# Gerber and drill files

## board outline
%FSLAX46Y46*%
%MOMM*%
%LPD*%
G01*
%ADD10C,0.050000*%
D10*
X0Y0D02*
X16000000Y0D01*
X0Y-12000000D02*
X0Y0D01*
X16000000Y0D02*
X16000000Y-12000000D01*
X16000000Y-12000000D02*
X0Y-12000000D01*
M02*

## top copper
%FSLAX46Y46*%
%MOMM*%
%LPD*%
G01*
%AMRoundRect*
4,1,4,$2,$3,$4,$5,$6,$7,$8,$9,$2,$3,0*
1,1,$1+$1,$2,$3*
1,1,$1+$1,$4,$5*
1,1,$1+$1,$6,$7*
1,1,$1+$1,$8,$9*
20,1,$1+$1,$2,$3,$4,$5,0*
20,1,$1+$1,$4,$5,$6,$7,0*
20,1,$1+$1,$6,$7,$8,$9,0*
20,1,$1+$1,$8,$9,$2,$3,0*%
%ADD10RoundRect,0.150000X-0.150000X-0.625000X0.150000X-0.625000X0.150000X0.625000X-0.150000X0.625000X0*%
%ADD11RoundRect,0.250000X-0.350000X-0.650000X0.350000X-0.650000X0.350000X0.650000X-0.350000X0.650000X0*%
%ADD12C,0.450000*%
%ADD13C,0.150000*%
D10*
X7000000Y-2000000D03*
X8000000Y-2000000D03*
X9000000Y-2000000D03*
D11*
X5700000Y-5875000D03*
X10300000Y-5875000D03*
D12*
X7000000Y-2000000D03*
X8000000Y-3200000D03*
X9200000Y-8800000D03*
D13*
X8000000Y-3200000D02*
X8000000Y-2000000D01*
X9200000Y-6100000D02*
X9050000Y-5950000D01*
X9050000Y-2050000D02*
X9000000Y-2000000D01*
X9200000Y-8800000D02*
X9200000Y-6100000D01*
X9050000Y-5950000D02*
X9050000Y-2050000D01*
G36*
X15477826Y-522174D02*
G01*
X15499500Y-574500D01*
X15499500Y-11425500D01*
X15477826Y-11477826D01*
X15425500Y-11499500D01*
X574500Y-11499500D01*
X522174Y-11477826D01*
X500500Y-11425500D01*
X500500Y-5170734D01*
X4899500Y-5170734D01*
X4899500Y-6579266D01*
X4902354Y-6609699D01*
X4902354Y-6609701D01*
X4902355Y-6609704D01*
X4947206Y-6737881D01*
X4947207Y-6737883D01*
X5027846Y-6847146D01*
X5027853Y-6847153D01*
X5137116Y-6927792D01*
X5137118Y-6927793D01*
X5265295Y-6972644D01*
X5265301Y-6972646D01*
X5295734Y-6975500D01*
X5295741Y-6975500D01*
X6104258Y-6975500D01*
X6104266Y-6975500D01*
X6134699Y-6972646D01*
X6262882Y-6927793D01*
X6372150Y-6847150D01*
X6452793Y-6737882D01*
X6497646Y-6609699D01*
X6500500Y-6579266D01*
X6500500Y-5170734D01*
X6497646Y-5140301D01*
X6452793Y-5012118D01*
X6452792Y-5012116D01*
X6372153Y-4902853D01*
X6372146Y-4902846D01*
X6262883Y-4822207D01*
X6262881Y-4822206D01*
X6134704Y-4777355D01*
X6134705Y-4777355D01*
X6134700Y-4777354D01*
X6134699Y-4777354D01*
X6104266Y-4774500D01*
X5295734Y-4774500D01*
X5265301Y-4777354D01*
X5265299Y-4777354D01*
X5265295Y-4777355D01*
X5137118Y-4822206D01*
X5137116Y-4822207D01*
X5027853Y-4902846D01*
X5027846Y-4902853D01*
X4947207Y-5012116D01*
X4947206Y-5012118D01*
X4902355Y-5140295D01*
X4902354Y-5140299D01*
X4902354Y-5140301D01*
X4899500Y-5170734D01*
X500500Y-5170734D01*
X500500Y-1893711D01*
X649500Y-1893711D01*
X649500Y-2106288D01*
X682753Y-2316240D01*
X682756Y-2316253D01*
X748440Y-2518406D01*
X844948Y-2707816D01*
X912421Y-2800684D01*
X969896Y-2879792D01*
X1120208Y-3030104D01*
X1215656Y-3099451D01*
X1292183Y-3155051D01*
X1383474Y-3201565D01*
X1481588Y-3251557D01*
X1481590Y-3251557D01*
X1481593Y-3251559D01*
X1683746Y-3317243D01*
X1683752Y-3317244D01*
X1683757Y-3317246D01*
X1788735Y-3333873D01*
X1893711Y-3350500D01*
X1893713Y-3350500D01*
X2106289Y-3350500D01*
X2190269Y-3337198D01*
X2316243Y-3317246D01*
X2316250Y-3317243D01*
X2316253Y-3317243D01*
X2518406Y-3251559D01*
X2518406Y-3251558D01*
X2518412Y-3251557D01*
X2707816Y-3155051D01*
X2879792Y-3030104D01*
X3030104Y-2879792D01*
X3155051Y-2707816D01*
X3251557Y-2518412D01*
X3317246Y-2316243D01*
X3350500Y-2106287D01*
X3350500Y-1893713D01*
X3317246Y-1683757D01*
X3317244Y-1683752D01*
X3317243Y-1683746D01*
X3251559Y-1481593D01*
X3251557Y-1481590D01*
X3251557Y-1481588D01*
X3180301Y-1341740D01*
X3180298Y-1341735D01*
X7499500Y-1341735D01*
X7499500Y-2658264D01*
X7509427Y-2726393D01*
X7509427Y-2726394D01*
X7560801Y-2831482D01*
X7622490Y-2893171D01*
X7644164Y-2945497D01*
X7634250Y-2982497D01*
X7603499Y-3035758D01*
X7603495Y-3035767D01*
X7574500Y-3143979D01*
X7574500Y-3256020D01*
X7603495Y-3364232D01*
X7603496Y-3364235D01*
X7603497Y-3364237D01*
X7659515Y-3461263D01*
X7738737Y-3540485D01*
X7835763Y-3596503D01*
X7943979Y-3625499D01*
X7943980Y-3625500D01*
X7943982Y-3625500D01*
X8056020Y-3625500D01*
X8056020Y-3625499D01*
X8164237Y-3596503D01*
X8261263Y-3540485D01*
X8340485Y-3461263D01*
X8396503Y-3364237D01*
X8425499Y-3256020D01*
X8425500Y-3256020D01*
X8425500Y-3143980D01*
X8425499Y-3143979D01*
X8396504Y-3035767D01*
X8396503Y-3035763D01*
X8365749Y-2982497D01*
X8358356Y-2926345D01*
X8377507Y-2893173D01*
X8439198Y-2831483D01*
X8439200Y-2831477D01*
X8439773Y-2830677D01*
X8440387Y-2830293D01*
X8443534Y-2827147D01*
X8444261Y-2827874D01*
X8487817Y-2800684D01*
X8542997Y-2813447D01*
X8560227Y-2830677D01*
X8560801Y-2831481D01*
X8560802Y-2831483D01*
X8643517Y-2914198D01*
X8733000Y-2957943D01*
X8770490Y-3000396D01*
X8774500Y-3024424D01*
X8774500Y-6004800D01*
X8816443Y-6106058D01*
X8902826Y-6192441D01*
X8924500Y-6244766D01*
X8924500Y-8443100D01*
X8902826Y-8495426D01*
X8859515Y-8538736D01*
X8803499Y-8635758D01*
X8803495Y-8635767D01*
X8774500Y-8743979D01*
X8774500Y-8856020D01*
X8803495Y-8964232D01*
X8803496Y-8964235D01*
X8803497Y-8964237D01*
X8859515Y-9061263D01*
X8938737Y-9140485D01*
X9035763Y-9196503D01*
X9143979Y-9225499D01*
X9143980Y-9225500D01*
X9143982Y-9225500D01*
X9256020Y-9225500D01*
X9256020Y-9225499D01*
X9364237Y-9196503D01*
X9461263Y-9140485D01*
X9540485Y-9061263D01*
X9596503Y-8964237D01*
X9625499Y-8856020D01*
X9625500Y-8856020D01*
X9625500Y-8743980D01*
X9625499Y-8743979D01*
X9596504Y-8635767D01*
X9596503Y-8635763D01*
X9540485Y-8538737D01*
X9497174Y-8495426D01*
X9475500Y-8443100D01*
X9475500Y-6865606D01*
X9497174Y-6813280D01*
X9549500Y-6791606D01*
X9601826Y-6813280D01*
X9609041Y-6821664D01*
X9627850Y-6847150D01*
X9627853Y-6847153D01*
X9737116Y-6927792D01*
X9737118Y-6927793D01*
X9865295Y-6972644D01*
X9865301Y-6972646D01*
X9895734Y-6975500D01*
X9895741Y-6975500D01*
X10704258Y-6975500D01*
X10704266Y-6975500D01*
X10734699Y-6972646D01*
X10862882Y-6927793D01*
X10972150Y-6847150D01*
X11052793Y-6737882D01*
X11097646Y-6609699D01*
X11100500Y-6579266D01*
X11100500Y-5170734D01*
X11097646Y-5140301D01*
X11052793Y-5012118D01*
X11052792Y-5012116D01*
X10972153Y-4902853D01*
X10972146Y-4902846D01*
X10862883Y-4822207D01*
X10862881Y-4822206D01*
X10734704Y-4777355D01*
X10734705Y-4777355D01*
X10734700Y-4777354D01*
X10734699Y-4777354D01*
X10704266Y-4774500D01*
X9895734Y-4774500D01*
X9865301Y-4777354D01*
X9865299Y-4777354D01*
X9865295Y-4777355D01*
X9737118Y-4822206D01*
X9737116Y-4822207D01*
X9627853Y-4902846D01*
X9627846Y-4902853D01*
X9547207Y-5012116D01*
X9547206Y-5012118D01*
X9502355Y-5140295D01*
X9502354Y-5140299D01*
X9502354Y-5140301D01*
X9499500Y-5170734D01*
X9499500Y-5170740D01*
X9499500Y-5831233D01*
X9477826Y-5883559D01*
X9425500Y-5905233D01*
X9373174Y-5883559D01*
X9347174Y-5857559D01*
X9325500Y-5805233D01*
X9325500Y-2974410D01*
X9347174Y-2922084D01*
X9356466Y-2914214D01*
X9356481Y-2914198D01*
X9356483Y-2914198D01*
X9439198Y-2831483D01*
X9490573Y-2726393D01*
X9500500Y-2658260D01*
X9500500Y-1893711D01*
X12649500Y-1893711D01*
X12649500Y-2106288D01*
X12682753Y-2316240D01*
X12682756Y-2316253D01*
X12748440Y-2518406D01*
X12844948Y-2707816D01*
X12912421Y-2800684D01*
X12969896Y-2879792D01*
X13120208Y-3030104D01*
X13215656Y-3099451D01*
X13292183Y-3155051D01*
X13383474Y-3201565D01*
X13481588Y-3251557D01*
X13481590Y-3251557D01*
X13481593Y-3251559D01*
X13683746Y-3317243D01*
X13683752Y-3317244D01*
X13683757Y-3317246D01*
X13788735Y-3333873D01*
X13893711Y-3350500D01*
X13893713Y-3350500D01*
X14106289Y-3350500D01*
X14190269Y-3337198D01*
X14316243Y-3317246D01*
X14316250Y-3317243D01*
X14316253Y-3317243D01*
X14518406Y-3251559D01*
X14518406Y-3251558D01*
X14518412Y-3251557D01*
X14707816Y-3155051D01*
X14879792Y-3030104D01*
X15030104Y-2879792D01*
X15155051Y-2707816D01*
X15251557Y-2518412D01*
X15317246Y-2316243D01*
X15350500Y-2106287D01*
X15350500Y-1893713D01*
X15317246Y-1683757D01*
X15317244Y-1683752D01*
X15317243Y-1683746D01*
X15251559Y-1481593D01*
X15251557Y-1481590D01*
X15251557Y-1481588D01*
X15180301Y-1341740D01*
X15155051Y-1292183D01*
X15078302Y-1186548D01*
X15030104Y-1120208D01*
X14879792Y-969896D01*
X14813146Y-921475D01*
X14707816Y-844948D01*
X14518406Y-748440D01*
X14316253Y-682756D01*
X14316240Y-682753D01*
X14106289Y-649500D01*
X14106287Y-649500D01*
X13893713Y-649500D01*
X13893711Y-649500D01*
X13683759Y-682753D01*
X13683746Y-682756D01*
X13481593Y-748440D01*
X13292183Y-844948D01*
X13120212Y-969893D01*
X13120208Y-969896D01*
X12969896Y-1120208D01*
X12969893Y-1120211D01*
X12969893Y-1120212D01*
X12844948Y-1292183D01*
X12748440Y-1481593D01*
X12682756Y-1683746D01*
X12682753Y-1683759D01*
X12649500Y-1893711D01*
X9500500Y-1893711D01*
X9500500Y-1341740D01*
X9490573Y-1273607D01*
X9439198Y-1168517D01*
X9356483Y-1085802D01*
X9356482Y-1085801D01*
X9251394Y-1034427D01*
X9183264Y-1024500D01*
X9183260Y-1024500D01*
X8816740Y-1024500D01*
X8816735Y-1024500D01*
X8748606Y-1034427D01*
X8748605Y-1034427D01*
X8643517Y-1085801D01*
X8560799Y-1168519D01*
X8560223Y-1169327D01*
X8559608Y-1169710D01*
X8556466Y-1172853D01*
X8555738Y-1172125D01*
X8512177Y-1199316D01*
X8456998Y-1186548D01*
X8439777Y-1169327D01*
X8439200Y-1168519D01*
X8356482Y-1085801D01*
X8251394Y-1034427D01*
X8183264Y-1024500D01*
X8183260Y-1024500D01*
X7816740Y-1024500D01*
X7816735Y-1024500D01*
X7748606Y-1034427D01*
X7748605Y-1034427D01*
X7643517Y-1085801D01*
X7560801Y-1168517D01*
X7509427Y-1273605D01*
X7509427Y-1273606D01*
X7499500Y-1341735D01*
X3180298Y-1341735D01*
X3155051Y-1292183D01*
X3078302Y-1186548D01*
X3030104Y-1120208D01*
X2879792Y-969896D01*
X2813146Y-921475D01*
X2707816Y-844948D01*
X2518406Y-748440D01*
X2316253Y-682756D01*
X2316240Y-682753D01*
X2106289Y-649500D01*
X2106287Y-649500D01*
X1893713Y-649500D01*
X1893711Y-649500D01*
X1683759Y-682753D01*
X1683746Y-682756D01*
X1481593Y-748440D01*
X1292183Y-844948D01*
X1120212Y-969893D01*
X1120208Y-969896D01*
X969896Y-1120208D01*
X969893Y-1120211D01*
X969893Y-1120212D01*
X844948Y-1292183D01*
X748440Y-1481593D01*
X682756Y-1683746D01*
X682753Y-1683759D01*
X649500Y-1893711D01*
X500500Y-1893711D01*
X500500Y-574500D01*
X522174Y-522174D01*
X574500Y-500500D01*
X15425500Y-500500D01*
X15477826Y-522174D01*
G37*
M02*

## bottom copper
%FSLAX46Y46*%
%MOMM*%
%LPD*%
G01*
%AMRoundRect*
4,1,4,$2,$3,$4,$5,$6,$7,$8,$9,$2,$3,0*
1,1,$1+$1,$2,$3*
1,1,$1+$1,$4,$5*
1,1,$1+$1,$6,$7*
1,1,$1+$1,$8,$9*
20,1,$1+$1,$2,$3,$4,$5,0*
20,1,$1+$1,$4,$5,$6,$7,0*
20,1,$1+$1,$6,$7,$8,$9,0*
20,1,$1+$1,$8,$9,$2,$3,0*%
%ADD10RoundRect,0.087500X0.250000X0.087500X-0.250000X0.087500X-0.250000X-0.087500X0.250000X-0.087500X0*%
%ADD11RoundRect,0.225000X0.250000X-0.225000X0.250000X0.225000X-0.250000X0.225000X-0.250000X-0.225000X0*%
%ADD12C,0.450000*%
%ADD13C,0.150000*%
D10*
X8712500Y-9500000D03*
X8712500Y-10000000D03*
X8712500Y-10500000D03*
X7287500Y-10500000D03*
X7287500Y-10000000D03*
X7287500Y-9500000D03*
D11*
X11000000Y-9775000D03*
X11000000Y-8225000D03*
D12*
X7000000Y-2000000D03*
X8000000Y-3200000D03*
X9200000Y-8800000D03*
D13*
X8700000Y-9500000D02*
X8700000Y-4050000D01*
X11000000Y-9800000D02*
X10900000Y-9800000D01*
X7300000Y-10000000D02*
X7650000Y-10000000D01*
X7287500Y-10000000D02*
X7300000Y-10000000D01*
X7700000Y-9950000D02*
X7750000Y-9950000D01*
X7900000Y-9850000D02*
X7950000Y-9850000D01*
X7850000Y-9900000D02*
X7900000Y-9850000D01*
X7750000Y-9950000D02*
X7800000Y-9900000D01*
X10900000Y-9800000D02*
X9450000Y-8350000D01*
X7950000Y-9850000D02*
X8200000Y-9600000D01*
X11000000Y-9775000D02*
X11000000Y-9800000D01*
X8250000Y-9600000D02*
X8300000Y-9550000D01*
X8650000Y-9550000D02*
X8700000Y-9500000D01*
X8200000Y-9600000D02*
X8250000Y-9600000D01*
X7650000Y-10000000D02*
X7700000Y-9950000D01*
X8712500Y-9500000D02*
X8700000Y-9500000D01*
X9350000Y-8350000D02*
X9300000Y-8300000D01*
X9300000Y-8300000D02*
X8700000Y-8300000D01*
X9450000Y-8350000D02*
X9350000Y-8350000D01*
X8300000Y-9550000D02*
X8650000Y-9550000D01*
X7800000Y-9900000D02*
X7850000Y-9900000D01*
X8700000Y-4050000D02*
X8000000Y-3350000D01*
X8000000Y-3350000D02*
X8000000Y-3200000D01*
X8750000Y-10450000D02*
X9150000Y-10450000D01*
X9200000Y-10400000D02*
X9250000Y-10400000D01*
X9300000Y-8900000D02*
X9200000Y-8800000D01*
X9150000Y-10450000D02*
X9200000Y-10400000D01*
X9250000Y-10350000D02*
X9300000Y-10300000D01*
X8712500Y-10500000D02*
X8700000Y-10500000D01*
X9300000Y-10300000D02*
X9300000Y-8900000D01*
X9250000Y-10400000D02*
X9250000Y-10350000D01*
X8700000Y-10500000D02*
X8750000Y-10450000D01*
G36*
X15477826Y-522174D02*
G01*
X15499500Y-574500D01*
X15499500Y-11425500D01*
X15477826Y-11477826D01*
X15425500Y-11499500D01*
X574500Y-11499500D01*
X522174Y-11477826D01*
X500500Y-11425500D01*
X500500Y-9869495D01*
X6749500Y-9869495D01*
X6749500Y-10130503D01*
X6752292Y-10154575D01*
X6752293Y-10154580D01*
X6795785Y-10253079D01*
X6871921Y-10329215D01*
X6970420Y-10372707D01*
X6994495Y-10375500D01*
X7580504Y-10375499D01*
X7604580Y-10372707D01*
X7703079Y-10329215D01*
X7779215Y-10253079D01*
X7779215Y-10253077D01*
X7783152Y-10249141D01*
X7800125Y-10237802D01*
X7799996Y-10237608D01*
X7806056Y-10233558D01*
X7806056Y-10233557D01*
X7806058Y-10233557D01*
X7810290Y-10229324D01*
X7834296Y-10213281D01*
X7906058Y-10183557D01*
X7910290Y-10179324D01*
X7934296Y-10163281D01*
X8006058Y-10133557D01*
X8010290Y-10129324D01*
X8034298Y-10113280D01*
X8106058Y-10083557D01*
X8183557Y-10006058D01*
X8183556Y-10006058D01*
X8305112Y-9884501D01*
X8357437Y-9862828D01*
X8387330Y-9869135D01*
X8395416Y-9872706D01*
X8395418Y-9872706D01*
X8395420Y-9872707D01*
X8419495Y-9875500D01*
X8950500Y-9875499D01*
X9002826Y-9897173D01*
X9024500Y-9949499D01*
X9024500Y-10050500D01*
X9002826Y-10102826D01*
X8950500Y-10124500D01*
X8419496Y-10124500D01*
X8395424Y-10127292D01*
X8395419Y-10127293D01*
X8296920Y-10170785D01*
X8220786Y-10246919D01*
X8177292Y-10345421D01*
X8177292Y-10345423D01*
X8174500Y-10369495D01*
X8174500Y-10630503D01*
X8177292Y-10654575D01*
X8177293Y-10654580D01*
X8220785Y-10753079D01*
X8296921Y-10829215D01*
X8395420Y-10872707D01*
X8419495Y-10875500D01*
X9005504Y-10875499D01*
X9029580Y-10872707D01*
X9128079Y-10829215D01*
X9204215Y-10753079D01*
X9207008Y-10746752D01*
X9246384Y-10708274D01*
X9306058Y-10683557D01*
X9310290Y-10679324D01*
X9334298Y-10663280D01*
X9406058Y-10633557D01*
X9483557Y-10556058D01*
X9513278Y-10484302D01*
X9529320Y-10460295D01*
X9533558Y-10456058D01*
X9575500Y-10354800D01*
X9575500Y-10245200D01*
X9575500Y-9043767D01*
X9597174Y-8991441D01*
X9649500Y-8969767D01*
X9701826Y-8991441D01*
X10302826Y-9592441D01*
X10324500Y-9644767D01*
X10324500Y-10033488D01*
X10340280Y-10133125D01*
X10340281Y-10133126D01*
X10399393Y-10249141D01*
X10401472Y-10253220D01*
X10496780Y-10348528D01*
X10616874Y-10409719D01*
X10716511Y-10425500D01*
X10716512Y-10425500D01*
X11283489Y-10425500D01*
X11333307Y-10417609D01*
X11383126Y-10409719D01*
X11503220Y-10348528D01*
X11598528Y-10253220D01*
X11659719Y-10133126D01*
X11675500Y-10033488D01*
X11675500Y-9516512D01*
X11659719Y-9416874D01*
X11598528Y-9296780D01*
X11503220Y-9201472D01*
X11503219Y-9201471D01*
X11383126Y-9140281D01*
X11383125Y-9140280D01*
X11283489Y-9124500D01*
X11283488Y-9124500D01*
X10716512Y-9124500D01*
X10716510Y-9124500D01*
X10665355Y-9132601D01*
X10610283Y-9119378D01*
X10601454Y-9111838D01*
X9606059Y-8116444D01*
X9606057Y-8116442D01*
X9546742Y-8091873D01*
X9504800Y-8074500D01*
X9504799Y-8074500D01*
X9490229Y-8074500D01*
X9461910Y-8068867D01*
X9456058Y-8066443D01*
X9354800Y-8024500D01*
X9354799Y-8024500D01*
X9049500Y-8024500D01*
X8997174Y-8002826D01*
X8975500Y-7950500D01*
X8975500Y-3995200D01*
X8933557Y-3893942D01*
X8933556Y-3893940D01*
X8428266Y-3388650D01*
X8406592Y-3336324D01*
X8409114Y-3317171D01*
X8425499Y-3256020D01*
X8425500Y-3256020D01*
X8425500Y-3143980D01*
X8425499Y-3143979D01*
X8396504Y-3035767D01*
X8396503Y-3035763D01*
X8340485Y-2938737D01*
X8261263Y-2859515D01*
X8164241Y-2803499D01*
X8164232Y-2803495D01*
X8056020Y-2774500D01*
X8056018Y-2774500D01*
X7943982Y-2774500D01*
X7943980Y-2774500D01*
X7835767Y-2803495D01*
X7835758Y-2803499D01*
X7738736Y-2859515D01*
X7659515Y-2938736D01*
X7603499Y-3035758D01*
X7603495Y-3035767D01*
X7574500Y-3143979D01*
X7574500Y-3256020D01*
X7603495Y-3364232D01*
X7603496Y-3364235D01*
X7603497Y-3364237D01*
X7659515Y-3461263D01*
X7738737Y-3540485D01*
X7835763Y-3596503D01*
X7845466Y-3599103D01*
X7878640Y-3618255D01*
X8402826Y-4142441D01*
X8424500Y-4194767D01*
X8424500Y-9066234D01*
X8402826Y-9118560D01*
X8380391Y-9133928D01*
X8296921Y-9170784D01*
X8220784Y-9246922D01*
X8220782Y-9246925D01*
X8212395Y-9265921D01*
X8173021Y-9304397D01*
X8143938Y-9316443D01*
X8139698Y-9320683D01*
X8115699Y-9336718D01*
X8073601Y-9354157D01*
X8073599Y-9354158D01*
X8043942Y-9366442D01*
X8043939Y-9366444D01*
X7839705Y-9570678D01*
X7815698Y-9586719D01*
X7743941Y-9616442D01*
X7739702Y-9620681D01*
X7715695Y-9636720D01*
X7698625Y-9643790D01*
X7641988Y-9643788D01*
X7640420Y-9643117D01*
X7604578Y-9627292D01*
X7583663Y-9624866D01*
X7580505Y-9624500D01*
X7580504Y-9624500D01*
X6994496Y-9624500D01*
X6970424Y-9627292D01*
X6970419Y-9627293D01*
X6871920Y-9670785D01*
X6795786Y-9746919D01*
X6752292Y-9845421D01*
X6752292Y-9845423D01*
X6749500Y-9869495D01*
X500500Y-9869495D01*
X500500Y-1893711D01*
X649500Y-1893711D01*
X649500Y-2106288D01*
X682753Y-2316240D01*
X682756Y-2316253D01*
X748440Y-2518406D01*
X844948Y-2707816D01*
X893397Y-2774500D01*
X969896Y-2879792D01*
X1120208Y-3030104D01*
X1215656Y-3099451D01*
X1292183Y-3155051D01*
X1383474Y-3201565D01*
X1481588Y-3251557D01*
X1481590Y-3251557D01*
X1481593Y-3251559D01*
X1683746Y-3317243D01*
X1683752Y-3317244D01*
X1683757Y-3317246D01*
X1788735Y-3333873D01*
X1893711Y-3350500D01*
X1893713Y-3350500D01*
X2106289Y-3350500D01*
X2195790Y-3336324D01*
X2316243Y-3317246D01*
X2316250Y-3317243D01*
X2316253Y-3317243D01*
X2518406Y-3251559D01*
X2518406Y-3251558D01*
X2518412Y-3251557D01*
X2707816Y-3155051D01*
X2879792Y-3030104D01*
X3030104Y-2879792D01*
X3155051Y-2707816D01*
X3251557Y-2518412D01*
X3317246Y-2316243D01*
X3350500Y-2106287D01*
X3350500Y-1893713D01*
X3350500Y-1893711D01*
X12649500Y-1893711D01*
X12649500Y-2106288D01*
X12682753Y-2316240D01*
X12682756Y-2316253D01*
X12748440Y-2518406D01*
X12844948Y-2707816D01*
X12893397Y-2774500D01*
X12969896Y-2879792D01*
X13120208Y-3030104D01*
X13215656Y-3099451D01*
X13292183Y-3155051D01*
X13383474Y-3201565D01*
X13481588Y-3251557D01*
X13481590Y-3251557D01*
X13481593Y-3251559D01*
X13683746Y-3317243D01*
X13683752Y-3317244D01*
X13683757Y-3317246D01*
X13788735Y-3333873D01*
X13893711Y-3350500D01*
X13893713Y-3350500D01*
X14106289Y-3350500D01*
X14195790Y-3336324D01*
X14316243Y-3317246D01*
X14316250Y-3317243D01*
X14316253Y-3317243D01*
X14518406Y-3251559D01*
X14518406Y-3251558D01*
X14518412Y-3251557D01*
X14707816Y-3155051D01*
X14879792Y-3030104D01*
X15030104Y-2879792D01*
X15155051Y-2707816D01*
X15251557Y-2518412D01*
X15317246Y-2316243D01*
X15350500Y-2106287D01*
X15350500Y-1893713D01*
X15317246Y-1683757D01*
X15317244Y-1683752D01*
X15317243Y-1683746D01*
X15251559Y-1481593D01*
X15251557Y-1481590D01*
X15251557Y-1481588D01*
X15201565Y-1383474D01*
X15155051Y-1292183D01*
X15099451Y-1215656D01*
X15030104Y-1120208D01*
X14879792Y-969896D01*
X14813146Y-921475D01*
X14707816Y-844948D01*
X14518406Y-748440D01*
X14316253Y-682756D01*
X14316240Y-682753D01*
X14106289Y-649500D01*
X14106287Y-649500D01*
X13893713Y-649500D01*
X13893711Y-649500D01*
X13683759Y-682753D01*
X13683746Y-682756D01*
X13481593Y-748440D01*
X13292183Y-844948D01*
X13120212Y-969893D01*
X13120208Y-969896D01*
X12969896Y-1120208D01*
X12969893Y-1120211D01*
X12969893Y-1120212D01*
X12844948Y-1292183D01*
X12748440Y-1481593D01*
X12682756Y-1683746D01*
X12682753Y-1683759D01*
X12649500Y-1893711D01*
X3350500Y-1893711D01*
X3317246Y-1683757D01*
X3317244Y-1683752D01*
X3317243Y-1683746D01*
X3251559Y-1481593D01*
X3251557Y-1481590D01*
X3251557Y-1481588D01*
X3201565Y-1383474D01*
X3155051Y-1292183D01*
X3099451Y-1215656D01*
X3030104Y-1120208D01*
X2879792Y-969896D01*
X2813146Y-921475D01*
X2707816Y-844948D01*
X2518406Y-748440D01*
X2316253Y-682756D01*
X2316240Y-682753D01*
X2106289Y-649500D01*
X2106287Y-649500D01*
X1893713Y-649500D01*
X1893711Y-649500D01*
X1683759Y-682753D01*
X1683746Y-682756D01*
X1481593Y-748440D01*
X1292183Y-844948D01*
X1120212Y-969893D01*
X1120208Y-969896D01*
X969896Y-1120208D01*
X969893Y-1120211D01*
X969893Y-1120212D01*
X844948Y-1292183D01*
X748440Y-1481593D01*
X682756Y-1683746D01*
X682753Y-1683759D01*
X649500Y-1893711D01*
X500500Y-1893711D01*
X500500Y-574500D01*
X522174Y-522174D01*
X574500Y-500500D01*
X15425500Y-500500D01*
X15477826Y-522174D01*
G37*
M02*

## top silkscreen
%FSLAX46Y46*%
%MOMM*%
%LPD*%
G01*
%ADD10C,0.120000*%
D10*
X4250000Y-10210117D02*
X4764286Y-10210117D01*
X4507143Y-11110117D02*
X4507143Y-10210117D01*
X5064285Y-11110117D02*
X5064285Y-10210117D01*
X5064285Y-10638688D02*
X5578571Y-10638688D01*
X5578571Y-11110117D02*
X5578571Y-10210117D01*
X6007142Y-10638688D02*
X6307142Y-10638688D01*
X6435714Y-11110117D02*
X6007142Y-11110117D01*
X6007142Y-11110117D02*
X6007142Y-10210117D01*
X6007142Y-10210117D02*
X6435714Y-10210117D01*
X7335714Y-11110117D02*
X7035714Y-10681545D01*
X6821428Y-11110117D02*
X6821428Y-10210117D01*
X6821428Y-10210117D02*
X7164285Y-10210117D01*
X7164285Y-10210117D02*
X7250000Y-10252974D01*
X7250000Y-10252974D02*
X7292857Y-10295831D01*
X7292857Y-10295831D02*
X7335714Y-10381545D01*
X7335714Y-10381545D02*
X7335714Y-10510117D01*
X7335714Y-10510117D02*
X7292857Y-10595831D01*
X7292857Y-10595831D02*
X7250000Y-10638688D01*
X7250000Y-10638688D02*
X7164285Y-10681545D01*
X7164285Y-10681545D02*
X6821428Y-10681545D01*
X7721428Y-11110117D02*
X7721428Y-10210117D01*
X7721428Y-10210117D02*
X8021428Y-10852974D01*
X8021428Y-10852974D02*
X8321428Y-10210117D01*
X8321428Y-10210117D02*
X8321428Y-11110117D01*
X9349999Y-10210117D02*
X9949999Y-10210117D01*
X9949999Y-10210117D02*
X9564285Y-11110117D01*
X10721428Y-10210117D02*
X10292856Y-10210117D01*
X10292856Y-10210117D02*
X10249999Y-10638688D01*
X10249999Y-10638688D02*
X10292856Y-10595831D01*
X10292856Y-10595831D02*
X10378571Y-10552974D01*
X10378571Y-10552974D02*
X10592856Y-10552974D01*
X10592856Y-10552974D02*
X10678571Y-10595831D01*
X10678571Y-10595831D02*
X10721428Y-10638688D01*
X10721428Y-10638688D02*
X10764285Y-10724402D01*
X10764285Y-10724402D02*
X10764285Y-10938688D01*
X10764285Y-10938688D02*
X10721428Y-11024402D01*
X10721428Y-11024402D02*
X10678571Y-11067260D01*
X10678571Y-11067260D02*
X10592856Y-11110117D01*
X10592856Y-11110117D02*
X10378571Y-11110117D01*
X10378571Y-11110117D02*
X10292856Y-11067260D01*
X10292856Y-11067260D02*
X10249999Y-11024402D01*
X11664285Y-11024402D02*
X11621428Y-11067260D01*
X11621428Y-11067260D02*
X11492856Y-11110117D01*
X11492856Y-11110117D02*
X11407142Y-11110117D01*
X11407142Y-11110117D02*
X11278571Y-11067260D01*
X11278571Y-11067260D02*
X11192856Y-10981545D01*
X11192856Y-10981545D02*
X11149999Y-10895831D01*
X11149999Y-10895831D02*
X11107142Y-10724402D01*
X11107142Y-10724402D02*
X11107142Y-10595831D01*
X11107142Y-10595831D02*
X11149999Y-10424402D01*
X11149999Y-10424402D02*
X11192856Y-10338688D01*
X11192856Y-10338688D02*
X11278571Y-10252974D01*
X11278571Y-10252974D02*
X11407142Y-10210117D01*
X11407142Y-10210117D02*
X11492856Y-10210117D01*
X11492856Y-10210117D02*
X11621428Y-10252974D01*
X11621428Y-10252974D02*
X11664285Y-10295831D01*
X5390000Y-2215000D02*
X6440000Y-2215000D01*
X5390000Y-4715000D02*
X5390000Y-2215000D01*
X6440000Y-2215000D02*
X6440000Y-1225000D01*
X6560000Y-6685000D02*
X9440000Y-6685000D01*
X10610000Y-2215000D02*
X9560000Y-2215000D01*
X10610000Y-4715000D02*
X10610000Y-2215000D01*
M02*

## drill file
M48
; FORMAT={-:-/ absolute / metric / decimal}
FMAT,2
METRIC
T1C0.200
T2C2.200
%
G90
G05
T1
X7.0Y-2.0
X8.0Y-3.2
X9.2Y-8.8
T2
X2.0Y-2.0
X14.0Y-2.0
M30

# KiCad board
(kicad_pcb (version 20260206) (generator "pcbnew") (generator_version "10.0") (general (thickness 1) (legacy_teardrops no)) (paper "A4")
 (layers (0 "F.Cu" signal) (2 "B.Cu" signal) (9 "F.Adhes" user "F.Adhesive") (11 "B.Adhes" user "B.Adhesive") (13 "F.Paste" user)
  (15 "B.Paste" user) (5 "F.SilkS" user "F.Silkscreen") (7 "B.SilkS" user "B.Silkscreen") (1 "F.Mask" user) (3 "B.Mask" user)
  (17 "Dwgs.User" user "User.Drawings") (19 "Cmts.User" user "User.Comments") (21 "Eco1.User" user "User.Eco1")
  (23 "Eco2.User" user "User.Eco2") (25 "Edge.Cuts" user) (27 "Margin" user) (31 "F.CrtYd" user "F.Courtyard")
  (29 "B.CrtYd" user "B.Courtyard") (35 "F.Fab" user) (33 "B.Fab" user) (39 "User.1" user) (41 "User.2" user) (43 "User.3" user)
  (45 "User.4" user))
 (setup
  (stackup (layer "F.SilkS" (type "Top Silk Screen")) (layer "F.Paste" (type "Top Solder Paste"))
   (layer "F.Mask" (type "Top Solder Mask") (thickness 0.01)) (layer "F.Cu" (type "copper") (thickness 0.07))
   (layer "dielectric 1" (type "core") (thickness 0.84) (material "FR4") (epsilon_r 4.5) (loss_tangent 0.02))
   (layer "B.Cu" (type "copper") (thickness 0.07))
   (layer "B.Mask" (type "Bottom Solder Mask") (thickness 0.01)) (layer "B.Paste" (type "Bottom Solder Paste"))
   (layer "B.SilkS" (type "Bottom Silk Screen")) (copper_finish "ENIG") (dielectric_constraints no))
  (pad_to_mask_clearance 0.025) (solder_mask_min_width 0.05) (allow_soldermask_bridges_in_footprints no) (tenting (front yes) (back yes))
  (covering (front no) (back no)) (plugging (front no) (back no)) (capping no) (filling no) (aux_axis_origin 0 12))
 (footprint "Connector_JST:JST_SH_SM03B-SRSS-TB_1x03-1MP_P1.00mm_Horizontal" (layer "F.Cu") (at 8 4)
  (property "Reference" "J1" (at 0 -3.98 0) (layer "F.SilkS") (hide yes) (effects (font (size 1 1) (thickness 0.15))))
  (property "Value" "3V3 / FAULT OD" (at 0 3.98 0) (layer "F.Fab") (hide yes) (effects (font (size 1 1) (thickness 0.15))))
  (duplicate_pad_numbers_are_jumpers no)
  (fp_line (start -2.61 -1.785) (end -1.56 -1.785) (stroke (width 0.12) (type solid)) (layer "F.SilkS"))
  (fp_line (start -2.61 0.715) (end -2.61 -1.785) (stroke (width 0.12) (type solid)) (layer "F.SilkS"))
  (fp_line (start -1.56 -1.785) (end -1.56 -2.775) (stroke (width 0.12) (type solid)) (layer "F.SilkS"))
  (fp_line (start -1.44 2.685) (end 1.44 2.685) (stroke (width 0.12) (type solid)) (layer "F.SilkS"))
  (fp_line (start 2.61 -1.785) (end 1.56 -1.785) (stroke (width 0.12) (type solid)) (layer "F.SilkS"))
  (fp_line (start 2.61 0.715) (end 2.61 -1.785) (stroke (width 0.12) (type solid)) (layer "F.SilkS"))
  (pad "1" smd roundrect (at -1 -2) (size 0.6 1.55) (layers "F.Cu" "F.Mask" "F.Paste") (roundrect_rratio 0.25) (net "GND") (zone_connect 2))
  (pad "2" smd roundrect (at 0 -2) (size 0.6 1.55) (layers "F.Cu" "F.Mask" "F.Paste") (roundrect_rratio 0.25) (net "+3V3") (zone_connect 2))
  (pad "3" smd roundrect (at 1 -2) (size 0.6 1.55) (layers "F.Cu" "F.Mask" "F.Paste") (roundrect_rratio 0.25) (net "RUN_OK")
   (zone_connect 2))
  (pad "MP" smd roundrect (at -2.3 1.875) (size 1.2 1.8) (layers "F.Cu" "F.Mask" "F.Paste") (roundrect_rratio 0.208333) (zone_connect 2))
  (pad "MP" smd roundrect (at 2.3 1.875) (size 1.2 1.8) (layers "F.Cu" "F.Mask" "F.Paste") (roundrect_rratio 0.208333) (zone_connect 2)))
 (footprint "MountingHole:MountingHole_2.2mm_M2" (layer "F.Cu") (at 2 2)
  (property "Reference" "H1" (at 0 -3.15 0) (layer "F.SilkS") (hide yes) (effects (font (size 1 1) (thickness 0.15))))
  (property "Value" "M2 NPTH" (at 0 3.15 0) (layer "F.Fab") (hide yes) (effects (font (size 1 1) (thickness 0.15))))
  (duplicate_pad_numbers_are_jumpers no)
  (pad "" np_thru_hole circle (at 0 0) (size 2.2 2.2) (drill 2.2) (layers "*.Cu" "*.Mask") (zone_connect 2)))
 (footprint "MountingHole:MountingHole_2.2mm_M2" (layer "F.Cu") (at 14 2)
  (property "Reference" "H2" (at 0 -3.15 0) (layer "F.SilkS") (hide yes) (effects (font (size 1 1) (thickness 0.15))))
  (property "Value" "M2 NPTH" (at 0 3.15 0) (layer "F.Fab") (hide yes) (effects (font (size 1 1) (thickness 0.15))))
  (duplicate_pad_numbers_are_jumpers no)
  (pad "" np_thru_hole circle (at 0 0) (size 2.2 2.2) (drill 2.2) (layers "*.Cu" "*.Mask") (zone_connect 2)))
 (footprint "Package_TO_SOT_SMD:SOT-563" (layer "B.Cu") (at 8 10 180)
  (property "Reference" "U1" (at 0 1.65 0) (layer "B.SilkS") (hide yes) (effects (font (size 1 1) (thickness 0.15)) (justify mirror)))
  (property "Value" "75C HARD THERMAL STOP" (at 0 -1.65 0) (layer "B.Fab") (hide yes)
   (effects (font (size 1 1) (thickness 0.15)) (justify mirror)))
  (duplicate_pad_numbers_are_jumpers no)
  (pad "1" smd roundrect (at -0.7125 0.5 180) (size 0.675 0.35) (layers "B.Cu" "B.Mask" "B.Paste") (roundrect_rratio 0.25) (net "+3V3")
   (zone_connect 2))
  (pad "2" smd roundrect (at -0.7125 0 180) (size 0.675 0.35) (layers "B.Cu" "B.Mask" "B.Paste") (roundrect_rratio 0.25) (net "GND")
   (zone_connect 2))
  (pad "3" smd roundrect (at -0.7125 -0.5 180) (size 0.675 0.35) (layers "B.Cu" "B.Mask" "B.Paste") (roundrect_rratio 0.25) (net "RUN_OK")
   (zone_connect 2))
  (pad "4" smd roundrect (at 0.7125 -0.5 180) (size 0.675 0.35) (layers "B.Cu" "B.Mask" "B.Paste") (roundrect_rratio 0.25) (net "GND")
   (zone_connect 2))
  (pad "5" smd roundrect (at 0.7125 0 180) (size 0.675 0.35) (layers "B.Cu" "B.Mask" "B.Paste") (roundrect_rratio 0.25) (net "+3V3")
   (zone_connect 2))
  (pad "6" smd roundrect (at 0.7125 0.5 180) (size 0.675 0.35) (layers "B.Cu" "B.Mask" "B.Paste") (roundrect_rratio 0.25) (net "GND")
   (zone_connect 2)))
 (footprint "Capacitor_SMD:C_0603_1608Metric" (layer "B.Cu") (at 11 9 90)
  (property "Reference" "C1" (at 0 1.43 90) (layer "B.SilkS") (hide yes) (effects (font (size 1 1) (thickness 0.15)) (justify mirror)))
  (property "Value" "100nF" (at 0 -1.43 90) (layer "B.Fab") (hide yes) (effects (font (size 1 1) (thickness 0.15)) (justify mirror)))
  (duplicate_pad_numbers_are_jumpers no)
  (pad "1" smd roundrect (at -0.775 0 90) (size 0.9 0.95) (layers "B.Cu" "B.Mask" "B.Paste") (roundrect_rratio 0.25) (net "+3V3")
   (zone_connect 2))
  (pad "2" smd roundrect (at 0.775 0 90) (size 0.9 0.95) (layers "B.Cu" "B.Mask" "B.Paste") (roundrect_rratio 0.25) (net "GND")
   (zone_connect 2)))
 (gr_line (start 0 0) (end 16 0) (stroke (width 0.05) (type default)) (layer "Edge.Cuts"))
 (gr_line (start 0 12) (end 0 0) (stroke (width 0.05) (type default)) (layer "Edge.Cuts"))
 (gr_line (start 16 0) (end 16 12) (stroke (width 0.05) (type default)) (layer "Edge.Cuts"))
 (gr_line (start 16 12) (end 0 12) (stroke (width 0.05) (type default)) (layer "Edge.Cuts"))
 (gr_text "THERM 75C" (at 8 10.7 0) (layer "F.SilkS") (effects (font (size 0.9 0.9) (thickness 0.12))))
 (via (at 7 2) (size 0.45) (drill 0.2) (layers "F.Cu" "B.Cu") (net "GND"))
 (segment (start 8 3.2) (end 8 2) (width 0.15) (layer "F.Cu") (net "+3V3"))
 (via (at 8 3.2) (size 0.45) (drill 0.2) (layers "F.Cu" "B.Cu") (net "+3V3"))
 (segment (start 8.7 9.5) (end 8.7 4.05) (width 0.15) (layer "B.Cu") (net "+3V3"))
 (segment (start 11 9.8) (end 10.9 9.8) (width 0.15) (layer "B.Cu") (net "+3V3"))
 (segment (start 7.3 10) (end 7.65 10) (width 0.15) (layer "B.Cu") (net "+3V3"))
 (segment (start 7.2875 10) (end 7.3 10) (width 0.15) (layer "B.Cu") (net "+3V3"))
 (segment (start 7.7 9.95) (end 7.75 9.95) (width 0.15) (layer "B.Cu") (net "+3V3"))
 (segment (start 7.9 9.85) (end 7.95 9.85) (width 0.15) (layer "B.Cu") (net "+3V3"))
 (segment (start 7.85 9.9) (end 7.9 9.85) (width 0.15) (layer "B.Cu") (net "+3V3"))
 (segment (start 7.75 9.95) (end 7.8 9.9) (width 0.15) (layer "B.Cu") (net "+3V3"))
 (segment (start 10.9 9.8) (end 9.45 8.35) (width 0.15) (layer "B.Cu") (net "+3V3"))
 (segment (start 7.95 9.85) (end 8.2 9.6) (width 0.15) (layer "B.Cu") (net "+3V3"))
 (segment (start 11 9.775) (end 11 9.8) (width 0.15) (layer "B.Cu") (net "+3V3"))
 (segment (start 8.25 9.6) (end 8.3 9.55) (width 0.15) (layer "B.Cu") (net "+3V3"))
 (segment (start 8.65 9.55) (end 8.7 9.5) (width 0.15) (layer "B.Cu") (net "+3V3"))
 (segment (start 8.2 9.6) (end 8.25 9.6) (width 0.15) (layer "B.Cu") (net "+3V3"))
 (segment (start 7.65 10) (end 7.7 9.95) (width 0.15) (layer "B.Cu") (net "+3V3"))
 (segment (start 8.7125 9.5) (end 8.7 9.5) (width 0.15) (layer "B.Cu") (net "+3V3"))
 (segment (start 9.35 8.35) (end 9.3 8.3) (width 0.15) (layer "B.Cu") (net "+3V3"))
 (segment (start 9.3 8.3) (end 8.7 8.3) (width 0.15) (layer "B.Cu") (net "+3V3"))
 (segment (start 9.45 8.35) (end 9.35 8.35) (width 0.15) (layer "B.Cu") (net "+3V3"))
 (segment (start 8.3 9.55) (end 8.65 9.55) (width 0.15) (layer "B.Cu") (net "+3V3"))
 (segment (start 7.8 9.9) (end 7.85 9.9) (width 0.15) (layer "B.Cu") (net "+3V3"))
 (segment (start 8.7 4.05) (end 8 3.35) (width 0.15) (layer "B.Cu") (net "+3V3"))
 (segment (start 8 3.35) (end 8 3.2) (width 0.15) (layer "B.Cu") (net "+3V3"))
 (segment (start 9.2 6.1) (end 9.05 5.95) (width 0.15) (layer "F.Cu") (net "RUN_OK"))
 (segment (start 9.05 2.05) (end 9 2) (width 0.15) (layer "F.Cu") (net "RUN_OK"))
 (segment (start 9.2 8.8) (end 9.2 6.1) (width 0.15) (layer "F.Cu") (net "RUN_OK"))
 (segment (start 9.05 5.95) (end 9.05 2.05) (width 0.15) (layer "F.Cu") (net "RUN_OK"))
 (via (at 9.2 8.8) (size 0.45) (drill 0.2) (layers "F.Cu" "B.Cu") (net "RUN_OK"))
 (segment (start 8.75 10.45) (end 9.15 10.45) (width 0.15) (layer "B.Cu") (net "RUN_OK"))
 (segment (start 9.2 10.4) (end 9.25 10.4) (width 0.15) (layer "B.Cu") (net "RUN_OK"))
 (segment (start 9.3 8.9) (end 9.2 8.8) (width 0.15) (layer "B.Cu") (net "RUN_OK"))
 (segment (start 9.15 10.45) (end 9.2 10.4) (width 0.15) (layer "B.Cu") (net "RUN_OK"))
 (segment (start 9.25 10.35) (end 9.3 10.3) (width 0.15) (layer "B.Cu") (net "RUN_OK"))
 (segment (start 8.7125 10.5) (end 8.7 10.5) (width 0.15) (layer "B.Cu") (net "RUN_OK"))
 (segment (start 9.3 10.3) (end 9.3 8.9) (width 0.15) (layer "B.Cu") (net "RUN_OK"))
 (segment (start 9.25 10.4) (end 9.25 10.35) (width 0.15) (layer "B.Cu") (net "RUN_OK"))
 (segment (start 8.7 10.5) (end 8.75 10.45) (width 0.15) (layer "B.Cu") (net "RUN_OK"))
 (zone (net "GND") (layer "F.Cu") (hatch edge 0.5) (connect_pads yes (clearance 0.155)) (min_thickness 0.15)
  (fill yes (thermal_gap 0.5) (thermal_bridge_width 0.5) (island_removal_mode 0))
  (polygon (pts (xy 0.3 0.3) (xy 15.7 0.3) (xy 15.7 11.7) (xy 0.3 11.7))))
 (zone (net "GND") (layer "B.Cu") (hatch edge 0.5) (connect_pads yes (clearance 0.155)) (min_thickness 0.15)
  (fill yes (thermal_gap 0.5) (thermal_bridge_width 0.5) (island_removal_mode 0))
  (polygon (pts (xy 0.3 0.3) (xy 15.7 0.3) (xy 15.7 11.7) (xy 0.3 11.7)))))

